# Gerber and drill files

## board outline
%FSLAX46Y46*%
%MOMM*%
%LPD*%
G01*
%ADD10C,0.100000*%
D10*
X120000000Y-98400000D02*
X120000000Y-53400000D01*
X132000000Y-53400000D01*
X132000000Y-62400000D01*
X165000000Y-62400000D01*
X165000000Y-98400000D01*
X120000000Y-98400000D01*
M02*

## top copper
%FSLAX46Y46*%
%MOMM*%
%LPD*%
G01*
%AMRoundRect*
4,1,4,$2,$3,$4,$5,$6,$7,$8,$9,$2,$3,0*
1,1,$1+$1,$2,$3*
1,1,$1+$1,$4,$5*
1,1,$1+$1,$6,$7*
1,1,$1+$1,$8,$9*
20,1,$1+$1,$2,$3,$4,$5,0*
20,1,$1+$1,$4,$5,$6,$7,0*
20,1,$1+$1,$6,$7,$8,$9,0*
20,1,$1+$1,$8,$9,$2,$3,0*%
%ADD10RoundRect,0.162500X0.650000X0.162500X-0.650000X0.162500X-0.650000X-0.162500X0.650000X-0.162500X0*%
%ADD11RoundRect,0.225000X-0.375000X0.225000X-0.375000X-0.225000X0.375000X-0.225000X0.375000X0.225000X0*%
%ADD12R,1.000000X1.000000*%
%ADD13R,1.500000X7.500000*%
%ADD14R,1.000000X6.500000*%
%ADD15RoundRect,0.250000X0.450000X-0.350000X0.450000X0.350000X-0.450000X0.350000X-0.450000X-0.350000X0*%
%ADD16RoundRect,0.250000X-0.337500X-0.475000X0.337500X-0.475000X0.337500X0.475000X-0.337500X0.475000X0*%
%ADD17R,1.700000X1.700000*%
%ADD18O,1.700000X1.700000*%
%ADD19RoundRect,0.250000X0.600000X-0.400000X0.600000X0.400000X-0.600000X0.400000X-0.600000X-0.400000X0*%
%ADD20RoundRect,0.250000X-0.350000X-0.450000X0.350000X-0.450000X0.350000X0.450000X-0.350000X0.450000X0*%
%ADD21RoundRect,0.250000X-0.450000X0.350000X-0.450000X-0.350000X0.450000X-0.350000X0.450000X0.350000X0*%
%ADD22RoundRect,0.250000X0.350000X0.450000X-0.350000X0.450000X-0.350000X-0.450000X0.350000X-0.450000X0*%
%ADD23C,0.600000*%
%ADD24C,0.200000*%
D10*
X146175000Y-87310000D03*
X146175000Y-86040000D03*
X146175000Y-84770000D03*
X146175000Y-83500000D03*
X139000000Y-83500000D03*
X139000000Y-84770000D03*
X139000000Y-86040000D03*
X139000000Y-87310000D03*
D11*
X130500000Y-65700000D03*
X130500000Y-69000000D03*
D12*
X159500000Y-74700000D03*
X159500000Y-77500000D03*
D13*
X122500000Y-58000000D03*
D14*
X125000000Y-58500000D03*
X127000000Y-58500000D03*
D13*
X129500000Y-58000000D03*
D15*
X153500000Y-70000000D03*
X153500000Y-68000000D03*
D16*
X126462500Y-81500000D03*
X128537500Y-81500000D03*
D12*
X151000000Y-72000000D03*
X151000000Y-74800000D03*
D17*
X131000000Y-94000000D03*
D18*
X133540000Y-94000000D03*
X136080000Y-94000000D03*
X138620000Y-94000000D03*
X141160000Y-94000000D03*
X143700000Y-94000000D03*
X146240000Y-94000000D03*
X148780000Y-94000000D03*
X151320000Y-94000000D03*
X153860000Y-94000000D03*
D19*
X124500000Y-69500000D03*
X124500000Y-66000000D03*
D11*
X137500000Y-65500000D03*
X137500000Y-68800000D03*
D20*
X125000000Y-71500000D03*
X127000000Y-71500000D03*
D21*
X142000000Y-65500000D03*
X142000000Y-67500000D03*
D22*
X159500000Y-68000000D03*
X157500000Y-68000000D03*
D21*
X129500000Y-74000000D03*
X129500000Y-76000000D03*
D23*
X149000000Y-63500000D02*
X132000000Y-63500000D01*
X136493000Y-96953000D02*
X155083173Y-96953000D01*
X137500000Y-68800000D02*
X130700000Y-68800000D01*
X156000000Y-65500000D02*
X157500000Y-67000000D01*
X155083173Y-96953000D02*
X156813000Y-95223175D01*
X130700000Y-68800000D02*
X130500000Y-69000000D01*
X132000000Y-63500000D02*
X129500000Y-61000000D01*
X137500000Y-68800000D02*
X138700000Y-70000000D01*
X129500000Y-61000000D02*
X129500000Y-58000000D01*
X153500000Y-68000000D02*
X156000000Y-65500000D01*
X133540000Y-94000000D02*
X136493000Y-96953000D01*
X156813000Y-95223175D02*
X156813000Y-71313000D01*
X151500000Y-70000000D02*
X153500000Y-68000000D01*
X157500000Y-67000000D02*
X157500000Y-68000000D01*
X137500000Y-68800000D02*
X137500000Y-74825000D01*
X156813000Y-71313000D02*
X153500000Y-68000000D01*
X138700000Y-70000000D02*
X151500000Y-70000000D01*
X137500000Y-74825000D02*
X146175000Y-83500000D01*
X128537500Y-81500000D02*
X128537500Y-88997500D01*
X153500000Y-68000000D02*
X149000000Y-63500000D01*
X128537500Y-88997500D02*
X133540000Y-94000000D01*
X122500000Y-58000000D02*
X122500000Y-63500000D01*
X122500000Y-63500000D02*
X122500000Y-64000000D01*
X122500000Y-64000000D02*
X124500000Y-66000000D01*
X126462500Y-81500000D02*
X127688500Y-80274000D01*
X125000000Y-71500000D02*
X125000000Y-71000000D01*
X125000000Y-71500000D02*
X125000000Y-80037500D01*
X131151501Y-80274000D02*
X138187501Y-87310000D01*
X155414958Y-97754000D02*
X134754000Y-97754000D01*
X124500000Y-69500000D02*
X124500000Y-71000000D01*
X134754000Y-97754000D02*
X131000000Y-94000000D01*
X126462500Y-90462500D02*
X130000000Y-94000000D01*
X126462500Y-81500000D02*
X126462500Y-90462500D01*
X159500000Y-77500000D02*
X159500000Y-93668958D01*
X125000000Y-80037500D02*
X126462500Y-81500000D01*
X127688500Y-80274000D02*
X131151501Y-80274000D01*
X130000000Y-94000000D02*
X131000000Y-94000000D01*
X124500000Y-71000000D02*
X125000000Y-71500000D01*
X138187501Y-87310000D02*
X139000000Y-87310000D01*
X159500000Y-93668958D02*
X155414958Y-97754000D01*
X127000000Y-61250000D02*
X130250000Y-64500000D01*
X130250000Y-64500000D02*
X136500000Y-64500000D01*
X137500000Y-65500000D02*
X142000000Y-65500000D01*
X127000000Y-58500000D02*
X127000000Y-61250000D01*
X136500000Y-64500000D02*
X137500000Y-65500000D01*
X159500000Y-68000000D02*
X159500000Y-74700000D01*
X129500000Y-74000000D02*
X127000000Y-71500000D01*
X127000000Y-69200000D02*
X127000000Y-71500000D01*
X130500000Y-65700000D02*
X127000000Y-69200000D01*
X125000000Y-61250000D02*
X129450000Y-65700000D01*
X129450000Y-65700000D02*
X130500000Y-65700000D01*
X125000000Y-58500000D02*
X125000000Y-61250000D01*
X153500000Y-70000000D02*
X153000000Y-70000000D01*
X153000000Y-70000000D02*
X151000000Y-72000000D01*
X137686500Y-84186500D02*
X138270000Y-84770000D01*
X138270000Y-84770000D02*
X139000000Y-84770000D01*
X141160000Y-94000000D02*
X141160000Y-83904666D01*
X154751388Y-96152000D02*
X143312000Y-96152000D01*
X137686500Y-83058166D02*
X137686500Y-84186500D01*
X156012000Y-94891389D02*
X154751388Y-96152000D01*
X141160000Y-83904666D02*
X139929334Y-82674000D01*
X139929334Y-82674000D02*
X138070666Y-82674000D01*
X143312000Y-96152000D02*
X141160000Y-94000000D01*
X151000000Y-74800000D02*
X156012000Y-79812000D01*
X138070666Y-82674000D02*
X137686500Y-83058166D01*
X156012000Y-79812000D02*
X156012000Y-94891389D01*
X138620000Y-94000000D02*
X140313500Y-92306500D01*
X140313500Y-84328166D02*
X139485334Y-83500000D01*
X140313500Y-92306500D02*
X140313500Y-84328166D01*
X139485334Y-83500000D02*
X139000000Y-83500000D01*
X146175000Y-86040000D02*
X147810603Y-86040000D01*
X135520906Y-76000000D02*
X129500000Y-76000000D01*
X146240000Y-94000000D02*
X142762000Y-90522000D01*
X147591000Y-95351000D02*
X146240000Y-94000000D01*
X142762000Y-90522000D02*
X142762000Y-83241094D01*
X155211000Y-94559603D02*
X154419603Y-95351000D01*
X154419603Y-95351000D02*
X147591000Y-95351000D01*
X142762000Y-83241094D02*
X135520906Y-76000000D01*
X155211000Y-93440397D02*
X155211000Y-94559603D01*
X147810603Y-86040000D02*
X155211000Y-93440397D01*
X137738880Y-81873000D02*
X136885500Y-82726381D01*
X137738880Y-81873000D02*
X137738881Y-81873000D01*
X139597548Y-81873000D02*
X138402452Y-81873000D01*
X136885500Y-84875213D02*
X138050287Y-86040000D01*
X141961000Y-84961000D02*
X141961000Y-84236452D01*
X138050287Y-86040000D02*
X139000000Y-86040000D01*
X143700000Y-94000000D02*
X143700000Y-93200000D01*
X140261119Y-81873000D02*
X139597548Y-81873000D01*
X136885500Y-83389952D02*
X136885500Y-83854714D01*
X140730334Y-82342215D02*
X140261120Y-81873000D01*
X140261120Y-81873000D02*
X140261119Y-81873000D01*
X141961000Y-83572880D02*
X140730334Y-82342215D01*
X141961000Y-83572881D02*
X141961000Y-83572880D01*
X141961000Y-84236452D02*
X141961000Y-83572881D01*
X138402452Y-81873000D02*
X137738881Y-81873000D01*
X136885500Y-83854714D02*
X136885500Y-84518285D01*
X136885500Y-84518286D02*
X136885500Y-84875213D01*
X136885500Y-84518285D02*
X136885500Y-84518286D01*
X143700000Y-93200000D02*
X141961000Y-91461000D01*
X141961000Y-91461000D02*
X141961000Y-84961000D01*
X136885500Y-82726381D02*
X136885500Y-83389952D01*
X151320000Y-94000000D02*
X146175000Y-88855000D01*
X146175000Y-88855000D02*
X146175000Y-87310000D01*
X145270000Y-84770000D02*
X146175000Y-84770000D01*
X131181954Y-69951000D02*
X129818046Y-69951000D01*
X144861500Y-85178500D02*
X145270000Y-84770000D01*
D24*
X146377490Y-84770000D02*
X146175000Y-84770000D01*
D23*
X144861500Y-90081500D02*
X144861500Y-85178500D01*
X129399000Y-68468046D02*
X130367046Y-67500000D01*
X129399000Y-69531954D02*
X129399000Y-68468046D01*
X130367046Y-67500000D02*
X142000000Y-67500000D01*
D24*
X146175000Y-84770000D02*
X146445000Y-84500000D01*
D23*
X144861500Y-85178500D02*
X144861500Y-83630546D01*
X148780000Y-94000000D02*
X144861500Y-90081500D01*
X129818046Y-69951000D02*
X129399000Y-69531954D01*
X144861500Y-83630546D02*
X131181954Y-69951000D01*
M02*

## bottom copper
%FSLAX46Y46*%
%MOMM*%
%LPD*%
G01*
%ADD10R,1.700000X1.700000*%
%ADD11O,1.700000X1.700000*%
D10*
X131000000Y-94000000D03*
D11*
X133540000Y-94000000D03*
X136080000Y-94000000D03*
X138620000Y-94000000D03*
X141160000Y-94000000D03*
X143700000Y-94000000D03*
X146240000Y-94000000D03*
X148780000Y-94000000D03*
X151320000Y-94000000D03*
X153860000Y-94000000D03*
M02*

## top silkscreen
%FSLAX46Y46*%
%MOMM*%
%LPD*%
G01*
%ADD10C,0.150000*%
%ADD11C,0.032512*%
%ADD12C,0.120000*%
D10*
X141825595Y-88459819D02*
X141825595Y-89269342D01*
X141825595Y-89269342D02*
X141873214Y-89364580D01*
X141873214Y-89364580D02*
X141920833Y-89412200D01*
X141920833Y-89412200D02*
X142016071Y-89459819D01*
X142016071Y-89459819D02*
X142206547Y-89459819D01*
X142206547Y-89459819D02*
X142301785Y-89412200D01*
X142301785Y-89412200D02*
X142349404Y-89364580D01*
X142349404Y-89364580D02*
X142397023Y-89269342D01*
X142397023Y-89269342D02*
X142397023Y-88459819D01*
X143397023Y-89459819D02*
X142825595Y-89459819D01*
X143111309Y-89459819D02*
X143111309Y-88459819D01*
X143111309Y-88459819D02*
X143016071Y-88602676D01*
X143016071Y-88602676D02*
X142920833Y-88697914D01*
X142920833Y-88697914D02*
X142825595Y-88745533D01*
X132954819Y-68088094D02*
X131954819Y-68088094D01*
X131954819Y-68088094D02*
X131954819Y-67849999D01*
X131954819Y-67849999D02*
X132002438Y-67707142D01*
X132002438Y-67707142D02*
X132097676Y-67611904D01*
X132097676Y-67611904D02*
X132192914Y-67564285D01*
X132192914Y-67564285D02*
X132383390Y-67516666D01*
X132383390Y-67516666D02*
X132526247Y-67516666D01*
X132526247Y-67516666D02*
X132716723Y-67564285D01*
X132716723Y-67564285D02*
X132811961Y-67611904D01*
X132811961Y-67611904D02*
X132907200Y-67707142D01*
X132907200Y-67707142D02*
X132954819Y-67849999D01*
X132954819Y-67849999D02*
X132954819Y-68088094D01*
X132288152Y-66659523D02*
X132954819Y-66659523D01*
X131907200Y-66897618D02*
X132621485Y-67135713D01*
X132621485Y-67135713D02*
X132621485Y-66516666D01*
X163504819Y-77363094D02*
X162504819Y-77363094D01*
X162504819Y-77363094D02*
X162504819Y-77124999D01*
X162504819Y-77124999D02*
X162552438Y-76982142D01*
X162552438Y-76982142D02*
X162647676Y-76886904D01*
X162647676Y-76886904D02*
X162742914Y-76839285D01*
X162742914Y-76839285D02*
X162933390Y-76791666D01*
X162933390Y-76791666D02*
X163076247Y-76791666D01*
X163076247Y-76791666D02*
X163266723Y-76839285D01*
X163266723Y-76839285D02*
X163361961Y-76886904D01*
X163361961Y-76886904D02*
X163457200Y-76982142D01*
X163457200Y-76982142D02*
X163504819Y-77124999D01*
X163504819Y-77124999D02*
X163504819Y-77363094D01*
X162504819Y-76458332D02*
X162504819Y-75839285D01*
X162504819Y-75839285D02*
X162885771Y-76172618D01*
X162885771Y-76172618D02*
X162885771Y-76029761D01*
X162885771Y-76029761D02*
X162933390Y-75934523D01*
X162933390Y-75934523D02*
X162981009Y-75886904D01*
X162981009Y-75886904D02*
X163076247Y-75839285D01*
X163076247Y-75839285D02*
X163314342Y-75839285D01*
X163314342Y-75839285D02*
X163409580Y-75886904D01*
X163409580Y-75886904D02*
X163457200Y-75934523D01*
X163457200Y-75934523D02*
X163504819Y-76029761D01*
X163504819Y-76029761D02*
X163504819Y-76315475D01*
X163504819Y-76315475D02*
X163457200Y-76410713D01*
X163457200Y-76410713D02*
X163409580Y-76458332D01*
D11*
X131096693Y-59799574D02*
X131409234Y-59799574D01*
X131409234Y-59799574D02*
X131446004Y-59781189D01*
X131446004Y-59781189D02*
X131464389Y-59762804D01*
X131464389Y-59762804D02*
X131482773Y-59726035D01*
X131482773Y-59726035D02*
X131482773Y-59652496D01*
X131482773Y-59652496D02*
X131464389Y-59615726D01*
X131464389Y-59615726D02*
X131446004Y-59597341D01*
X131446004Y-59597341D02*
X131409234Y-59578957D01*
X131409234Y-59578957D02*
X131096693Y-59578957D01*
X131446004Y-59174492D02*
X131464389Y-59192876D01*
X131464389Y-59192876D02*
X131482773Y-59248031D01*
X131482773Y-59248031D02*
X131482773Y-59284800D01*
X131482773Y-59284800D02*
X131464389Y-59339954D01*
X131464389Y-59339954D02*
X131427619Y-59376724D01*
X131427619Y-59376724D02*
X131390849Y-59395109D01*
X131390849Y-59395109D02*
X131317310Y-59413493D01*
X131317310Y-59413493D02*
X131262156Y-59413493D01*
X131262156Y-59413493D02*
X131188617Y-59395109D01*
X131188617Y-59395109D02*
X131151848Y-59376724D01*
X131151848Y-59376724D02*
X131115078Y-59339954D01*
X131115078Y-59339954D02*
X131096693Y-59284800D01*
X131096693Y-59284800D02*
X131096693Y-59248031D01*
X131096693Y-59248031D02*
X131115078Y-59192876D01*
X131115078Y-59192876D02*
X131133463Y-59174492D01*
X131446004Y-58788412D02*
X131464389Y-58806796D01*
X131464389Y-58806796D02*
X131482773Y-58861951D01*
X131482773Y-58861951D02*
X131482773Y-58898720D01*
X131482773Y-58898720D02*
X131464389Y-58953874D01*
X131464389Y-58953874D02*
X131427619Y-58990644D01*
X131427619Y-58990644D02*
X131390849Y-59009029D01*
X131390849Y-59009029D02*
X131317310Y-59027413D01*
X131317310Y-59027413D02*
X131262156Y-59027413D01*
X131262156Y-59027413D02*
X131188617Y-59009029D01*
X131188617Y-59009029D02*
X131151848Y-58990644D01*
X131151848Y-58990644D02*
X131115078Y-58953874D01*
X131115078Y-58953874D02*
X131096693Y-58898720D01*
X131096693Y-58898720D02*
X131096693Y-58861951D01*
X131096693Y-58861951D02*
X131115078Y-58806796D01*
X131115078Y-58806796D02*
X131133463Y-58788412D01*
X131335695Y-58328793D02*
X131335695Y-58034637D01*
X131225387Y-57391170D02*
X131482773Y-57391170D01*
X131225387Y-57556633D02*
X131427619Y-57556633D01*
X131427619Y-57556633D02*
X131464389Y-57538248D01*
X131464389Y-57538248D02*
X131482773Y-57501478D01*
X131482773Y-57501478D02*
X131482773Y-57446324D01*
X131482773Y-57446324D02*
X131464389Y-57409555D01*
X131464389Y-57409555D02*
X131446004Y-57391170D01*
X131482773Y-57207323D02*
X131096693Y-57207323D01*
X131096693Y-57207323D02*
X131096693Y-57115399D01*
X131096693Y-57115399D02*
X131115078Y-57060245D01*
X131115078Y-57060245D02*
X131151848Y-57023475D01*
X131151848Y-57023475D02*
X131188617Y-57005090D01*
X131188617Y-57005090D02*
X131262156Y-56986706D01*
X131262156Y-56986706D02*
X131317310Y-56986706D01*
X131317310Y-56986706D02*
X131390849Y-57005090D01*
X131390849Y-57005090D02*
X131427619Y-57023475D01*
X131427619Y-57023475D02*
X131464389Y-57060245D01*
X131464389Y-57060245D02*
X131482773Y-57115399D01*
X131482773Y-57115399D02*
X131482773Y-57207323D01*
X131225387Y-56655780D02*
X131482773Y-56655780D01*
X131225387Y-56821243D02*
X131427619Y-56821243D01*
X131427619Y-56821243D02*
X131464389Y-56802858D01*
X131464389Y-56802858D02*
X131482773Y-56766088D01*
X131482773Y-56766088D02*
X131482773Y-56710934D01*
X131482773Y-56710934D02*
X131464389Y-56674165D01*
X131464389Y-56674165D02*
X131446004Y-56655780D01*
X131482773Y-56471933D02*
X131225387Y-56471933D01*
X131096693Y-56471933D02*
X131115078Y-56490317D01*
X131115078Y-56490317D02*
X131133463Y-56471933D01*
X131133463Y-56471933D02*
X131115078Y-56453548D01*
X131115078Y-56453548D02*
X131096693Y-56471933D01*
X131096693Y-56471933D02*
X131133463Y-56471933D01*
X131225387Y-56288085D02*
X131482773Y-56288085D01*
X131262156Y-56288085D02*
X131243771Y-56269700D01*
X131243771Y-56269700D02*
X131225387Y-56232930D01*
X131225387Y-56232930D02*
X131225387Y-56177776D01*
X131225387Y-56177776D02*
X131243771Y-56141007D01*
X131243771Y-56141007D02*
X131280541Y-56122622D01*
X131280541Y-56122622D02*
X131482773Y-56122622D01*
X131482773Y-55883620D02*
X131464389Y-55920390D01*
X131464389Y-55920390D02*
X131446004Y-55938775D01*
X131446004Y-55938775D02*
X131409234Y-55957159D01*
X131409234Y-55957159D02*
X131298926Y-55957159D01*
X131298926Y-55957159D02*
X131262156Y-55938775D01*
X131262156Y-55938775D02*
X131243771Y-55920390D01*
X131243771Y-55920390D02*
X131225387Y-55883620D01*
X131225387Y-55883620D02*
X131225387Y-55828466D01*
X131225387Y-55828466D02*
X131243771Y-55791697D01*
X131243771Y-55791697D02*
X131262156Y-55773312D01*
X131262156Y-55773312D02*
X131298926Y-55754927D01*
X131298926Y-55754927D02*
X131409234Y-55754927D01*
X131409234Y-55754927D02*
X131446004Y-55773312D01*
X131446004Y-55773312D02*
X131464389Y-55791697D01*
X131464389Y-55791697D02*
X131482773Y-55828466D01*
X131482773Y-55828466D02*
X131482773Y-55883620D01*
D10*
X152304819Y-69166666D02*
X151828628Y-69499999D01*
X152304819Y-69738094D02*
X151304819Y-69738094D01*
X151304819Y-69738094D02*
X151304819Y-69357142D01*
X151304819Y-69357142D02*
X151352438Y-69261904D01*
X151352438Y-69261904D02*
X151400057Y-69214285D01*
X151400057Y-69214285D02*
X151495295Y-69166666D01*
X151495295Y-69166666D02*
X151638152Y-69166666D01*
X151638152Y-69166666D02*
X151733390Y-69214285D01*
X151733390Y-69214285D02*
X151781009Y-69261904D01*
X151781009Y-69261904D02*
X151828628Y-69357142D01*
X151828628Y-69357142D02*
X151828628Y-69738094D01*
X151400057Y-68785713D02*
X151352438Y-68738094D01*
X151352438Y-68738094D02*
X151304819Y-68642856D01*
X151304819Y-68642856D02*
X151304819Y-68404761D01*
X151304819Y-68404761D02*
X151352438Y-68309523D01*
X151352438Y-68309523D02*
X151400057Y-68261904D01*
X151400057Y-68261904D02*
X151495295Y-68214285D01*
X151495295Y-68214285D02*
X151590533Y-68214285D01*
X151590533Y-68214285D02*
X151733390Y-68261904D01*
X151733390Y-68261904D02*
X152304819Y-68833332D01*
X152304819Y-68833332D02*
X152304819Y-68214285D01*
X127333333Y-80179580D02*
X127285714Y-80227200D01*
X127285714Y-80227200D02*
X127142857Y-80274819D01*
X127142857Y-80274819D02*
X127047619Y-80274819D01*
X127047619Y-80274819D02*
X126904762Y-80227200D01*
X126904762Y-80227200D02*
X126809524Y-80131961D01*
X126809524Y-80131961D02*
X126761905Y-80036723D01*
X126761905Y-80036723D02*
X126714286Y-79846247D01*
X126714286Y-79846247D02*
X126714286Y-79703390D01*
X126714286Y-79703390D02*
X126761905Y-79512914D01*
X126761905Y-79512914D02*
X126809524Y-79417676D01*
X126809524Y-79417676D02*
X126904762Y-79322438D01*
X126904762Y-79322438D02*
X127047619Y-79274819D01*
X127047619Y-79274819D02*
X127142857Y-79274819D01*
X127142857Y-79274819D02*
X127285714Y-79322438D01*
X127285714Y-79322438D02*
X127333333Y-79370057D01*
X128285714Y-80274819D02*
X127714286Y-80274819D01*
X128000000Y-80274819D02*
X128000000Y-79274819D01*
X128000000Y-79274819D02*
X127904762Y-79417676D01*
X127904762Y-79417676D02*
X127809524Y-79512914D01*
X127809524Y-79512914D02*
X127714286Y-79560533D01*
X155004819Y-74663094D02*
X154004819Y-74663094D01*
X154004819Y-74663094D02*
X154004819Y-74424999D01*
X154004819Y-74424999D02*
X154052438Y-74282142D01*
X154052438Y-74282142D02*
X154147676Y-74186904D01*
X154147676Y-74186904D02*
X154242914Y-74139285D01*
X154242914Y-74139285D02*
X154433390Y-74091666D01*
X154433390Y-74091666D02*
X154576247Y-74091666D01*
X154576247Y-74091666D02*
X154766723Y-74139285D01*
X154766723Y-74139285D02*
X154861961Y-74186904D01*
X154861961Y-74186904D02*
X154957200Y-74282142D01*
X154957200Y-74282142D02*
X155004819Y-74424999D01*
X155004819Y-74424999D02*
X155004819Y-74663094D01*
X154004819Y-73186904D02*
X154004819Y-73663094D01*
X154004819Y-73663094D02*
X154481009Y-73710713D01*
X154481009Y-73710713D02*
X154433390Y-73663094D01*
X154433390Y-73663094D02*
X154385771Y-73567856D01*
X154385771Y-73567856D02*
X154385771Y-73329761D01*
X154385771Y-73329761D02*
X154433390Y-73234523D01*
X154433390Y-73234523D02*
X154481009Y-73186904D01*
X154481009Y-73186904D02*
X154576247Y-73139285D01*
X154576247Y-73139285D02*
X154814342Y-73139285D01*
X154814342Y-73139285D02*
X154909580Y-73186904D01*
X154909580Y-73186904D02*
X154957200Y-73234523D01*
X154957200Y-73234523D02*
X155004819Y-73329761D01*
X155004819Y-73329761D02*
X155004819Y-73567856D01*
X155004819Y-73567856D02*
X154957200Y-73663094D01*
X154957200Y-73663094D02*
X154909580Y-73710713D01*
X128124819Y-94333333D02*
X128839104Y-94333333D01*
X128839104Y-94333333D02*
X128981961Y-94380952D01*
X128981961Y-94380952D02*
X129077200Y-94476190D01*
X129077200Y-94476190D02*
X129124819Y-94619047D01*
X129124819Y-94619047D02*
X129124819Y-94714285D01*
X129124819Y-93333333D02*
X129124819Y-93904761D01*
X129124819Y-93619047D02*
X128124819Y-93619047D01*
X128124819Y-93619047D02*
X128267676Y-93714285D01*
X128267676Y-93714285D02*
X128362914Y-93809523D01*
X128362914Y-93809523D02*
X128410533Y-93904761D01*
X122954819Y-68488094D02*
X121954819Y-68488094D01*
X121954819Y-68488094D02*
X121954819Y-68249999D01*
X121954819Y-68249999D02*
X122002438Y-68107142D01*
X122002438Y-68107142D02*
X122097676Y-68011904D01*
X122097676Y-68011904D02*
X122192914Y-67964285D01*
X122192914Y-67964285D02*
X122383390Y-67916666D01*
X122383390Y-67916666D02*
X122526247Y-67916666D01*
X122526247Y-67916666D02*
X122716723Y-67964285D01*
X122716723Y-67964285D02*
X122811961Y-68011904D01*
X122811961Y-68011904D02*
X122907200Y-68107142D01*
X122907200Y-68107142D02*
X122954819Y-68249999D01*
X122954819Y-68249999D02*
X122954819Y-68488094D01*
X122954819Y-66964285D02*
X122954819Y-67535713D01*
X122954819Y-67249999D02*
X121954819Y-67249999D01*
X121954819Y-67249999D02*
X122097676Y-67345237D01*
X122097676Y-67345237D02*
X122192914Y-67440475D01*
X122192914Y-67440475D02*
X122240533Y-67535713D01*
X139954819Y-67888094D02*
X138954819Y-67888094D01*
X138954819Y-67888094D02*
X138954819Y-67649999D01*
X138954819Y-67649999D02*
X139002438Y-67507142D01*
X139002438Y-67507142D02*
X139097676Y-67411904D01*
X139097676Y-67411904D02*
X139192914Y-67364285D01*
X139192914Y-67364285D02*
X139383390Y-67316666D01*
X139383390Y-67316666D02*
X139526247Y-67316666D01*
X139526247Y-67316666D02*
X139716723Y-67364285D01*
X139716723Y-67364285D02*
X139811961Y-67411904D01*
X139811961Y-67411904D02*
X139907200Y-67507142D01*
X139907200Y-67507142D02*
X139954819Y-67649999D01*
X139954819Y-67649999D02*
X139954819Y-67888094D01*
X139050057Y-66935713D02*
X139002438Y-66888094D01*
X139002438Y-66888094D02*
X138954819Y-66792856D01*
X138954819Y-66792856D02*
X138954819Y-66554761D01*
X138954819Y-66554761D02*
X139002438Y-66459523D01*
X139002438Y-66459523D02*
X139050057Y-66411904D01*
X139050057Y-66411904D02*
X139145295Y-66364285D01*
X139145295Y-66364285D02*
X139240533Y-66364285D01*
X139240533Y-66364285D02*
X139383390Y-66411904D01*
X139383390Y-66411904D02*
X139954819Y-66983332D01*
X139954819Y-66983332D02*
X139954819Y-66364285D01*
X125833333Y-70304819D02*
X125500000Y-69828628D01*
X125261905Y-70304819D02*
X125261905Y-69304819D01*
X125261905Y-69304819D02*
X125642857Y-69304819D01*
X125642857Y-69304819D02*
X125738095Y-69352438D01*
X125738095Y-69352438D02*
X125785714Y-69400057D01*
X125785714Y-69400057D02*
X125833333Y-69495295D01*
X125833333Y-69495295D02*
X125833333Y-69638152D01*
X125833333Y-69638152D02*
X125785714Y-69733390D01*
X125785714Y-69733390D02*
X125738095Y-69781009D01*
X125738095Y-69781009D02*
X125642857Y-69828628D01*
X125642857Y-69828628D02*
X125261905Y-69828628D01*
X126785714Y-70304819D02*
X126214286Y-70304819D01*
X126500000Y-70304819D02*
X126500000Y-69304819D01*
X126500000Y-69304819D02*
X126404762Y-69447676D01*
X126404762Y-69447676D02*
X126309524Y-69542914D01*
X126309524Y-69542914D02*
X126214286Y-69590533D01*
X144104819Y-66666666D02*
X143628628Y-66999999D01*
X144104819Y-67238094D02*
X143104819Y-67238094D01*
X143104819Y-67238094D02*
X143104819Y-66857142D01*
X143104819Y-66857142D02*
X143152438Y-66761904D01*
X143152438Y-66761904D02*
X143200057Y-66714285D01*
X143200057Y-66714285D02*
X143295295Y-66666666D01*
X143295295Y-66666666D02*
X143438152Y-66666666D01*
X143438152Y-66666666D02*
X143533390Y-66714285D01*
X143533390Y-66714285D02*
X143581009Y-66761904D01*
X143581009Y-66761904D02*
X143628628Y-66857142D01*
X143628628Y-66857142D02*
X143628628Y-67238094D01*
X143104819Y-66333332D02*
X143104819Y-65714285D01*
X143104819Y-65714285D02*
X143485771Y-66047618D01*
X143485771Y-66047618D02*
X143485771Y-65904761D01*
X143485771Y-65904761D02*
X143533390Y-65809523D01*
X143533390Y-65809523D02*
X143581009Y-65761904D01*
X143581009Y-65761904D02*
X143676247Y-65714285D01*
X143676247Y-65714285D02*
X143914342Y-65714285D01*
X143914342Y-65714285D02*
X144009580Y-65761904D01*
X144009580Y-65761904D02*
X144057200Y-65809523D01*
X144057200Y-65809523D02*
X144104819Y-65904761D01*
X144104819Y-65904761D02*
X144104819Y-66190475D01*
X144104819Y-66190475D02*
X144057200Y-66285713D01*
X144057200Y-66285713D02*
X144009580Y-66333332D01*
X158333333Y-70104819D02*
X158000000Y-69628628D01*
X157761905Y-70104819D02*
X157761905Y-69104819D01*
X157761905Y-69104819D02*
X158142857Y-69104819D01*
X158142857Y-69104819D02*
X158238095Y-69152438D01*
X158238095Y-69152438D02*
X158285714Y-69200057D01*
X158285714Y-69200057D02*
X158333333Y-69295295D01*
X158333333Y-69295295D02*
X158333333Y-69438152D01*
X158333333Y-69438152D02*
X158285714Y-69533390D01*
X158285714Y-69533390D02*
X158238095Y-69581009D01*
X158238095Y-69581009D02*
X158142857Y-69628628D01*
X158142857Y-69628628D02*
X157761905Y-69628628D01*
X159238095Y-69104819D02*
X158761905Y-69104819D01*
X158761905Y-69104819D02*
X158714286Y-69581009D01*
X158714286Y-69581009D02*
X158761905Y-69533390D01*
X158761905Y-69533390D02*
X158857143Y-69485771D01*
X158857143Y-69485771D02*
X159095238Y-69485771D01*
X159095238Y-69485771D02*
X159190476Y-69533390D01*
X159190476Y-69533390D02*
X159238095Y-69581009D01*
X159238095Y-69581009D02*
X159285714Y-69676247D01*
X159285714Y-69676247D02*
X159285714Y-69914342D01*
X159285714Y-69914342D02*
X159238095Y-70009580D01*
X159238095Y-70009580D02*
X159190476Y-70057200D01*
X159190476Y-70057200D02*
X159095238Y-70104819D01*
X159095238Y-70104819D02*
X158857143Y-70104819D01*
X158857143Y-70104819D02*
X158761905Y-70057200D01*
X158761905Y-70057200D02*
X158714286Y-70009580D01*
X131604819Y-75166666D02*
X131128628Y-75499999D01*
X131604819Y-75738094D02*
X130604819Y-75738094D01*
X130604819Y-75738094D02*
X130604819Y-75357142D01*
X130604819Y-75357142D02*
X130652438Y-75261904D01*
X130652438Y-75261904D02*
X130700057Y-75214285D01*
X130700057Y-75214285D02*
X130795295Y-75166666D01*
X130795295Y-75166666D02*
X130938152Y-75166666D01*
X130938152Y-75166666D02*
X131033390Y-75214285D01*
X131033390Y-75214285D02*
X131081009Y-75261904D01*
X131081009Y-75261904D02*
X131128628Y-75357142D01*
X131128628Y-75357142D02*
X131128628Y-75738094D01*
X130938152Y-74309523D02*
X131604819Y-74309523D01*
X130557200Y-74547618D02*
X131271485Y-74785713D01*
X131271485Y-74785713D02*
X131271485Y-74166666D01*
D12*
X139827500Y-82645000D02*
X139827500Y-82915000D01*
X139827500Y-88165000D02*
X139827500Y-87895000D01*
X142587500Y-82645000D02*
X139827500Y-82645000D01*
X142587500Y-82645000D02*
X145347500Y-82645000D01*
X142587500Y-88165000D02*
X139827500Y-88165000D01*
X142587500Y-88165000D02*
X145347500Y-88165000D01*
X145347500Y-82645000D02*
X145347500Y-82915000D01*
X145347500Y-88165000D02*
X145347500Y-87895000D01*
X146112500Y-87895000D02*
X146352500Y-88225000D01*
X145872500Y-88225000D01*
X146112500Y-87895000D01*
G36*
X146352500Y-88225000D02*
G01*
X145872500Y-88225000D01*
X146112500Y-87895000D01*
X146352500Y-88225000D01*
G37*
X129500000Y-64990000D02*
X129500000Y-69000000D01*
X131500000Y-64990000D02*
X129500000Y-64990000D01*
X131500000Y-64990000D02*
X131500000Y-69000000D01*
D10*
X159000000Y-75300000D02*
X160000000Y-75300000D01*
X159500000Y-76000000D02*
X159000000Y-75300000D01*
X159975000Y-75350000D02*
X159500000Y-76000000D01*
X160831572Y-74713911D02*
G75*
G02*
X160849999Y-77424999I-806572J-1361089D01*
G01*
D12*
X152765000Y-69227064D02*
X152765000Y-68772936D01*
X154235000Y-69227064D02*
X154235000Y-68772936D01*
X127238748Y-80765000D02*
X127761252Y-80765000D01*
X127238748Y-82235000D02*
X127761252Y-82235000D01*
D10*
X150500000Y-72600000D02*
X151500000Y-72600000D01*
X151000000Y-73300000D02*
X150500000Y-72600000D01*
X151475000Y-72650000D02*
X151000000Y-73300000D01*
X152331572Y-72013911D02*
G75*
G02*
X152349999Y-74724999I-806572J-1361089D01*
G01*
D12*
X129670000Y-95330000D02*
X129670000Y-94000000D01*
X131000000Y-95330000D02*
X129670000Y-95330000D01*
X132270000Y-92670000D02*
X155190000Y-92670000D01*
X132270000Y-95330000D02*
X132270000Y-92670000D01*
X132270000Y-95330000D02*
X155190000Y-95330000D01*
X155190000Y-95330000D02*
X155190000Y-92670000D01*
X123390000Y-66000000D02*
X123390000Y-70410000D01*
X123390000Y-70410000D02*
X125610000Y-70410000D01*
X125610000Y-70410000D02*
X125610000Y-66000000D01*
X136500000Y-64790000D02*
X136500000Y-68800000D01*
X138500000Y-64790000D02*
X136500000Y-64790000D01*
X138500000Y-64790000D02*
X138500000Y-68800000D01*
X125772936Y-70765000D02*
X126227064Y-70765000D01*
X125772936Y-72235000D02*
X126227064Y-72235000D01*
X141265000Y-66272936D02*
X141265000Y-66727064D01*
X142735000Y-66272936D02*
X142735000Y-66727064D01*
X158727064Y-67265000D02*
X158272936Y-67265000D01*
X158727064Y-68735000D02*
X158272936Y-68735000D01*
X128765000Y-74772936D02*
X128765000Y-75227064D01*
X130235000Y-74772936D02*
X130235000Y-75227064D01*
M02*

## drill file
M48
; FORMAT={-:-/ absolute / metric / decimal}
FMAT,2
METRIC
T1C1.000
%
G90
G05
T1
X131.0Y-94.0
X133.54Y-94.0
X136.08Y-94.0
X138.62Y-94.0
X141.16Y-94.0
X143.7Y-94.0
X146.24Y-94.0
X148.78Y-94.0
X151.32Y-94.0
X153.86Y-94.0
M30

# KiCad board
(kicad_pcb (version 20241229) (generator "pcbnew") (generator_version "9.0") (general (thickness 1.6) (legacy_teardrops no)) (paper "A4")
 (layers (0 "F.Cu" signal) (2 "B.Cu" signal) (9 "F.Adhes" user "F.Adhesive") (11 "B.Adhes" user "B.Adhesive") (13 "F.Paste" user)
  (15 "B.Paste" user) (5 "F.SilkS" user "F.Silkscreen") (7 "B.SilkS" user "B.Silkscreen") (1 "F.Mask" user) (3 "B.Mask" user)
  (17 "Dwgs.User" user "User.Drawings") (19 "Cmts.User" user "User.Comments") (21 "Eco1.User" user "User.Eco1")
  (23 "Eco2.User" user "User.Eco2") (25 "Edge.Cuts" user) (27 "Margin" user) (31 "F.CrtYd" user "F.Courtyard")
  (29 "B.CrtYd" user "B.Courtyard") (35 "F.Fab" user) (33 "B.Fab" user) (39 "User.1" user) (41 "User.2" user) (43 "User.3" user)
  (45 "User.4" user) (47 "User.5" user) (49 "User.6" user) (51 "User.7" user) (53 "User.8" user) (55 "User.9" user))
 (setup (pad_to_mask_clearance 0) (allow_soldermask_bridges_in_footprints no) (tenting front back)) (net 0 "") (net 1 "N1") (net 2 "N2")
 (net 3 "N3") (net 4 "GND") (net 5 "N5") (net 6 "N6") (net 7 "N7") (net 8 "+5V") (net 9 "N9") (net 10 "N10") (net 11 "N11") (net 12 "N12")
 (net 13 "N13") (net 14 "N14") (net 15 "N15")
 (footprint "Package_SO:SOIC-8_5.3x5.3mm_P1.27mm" (layer "F.Cu") (at 142.5875 85.405 180)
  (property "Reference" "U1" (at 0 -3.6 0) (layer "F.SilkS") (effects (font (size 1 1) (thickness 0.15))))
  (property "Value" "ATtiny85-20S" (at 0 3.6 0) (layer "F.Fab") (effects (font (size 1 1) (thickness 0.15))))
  (fp_line (start 2.76 2.76) (end 2.76 2.49) (stroke (width 0.12) (type solid)) (layer "F.SilkS"))
  (fp_line (start 2.76 -2.76) (end 2.76 -2.49) (stroke (width 0.12) (type solid)) (layer "F.SilkS"))
  (fp_line (start 0 2.76) (end 2.76 2.76) (stroke (width 0.12) (type solid)) (layer "F.SilkS"))
  (fp_line (start 0 2.76) (end -2.76 2.76) (stroke (width 0.12) (type solid)) (layer "F.SilkS"))
  (fp_line (start 0 -2.76) (end 2.76 -2.76) (stroke (width 0.12) (type solid)) (layer "F.SilkS"))
  (fp_line (start 0 -2.76) (end -2.76 -2.76) (stroke (width 0.12) (type solid)) (layer "F.SilkS"))
  (fp_line (start -2.76 2.76) (end -2.76 2.49) (stroke (width 0.12) (type solid)) (layer "F.SilkS"))
  (fp_line (start -2.76 -2.76) (end -2.76 -2.49) (stroke (width 0.12) (type solid)) (layer "F.SilkS"))
  (fp_poly (pts (xy -3.525 -2.49) (xy -3.765 -2.82) (xy -3.285 -2.82)) (stroke (width 0.12) (type solid)) (fill yes) (layer "F.SilkS"))
  (pad "1" smd roundrect (at -3.5875 -1.905 180) (size 1.625 0.65) (layers "F.Cu" "F.Mask" "F.Paste") (roundrect_rratio 0.25) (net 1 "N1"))
  (pad "2" smd roundrect (at -3.5875 -0.635 180) (size 1.625 0.65) (layers "F.Cu" "F.Mask" "F.Paste") (roundrect_rratio 0.25) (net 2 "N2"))
  (pad "3" smd roundrect (at -3.5875 0.635 180) (size 1.625 0.65) (layers "F.Cu" "F.Mask" "F.Paste") (roundrect_rratio 0.25) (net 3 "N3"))
  (pad "4" smd roundrect (at -3.5875 1.905 180) (size 1.625 0.65) (layers "F.Cu" "F.Mask" "F.Paste") (roundrect_rratio 0.25) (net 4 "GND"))
  (pad "5" smd roundrect (at 3.5875 1.905 180) (size 1.625 0.65) (layers "F.Cu" "F.Mask" "F.Paste") (roundrect_rratio 0.25) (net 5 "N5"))
  (pad "6" smd roundrect (at 3.5875 0.635 180) (size 1.625 0.65) (layers "F.Cu" "F.Mask" "F.Paste") (roundrect_rratio 0.25) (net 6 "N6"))
  (pad "7" smd roundrect (at 3.5875 -0.635 180) (size 1.625 0.65) (layers "F.Cu" "F.Mask" "F.Paste") (roundrect_rratio 0.25) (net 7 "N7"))
  (pad "8" smd roundrect (at 3.5875 -1.905 180) (size 1.625 0.65) (layers "F.Cu" "F.Mask" "F.Paste") (roundrect_rratio 0.25) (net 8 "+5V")))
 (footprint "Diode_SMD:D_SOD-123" (layer "F.Cu") (at 130.5 67.35 -90)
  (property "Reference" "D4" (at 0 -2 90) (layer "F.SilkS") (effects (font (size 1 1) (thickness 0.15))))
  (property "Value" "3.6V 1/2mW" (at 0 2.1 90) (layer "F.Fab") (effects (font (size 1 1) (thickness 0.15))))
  (fp_line (start -2.36 1) (end 1.65 1) (stroke (width 0.12) (type solid)) (layer "F.SilkS"))
  (fp_line (start -2.36 -1) (end -2.36 1) (stroke (width 0.12) (type solid)) (layer "F.SilkS"))
  (fp_line (start -2.36 -1) (end 1.65 -1) (stroke (width 0.12) (type solid)) (layer "F.SilkS"))
  (pad "1" smd roundrect (at -1.65 0 270) (size 0.9 1.2) (layers "F.Cu" "F.Mask" "F.Paste") (roundrect_rratio 0.25) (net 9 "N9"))
  (pad "2" smd roundrect (at 1.65 0 270) (size 0.9 1.2) (layers "F.Cu" "F.Mask" "F.Paste") (roundrect_rratio 0.25) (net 4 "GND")))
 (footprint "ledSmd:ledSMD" (layer "F.Cu") (at 159.5 76.5 -90)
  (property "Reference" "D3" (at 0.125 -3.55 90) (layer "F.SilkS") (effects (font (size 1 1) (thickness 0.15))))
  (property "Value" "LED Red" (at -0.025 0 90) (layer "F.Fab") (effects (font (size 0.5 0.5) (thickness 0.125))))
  (fp_line (start -1.2 0.5) (end -1.2 -0.5) (stroke (width 0.15) (type solid)) (layer "F.SilkS"))
  (fp_line (start -0.5 0) (end -1.2 0.5) (stroke (width 0.15) (type solid)) (layer "F.SilkS"))
  (fp_line (start -1.15 -0.475) (end -0.5 0) (stroke (width 0.15) (type solid)) (layer "F.SilkS"))
  (fp_arc (start -1.786089 -1.331572) (mid -0.435753 -2.107089) (end 0.924999 -1.349999) (stroke (width 0.15) (type solid))
   (layer "F.SilkS"))
  (pad "1" smd rect (at -1.8 0 270) (size 1 1) (layers "F.Cu" "F.Mask" "F.Paste") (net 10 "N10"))
  (pad "2" smd rect (at 1 0 270) (size 1 1) (layers "F.Cu" "F.Mask" "F.Paste") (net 8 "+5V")))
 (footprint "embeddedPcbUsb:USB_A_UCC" (layer "F.Cu") (at 126 58.2 -90)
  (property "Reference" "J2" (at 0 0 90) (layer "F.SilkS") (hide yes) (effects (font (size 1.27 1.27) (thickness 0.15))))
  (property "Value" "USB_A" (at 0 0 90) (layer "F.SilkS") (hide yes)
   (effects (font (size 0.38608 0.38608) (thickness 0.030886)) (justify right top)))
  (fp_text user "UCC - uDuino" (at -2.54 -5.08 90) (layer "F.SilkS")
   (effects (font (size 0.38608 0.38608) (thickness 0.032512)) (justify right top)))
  (pad "1" smd rect (at -0.2 3.5 270) (size 7.5 1.5) (layers "F.Cu" "F.Mask" "F.Paste") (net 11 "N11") (solder_mask_margin 0.1016))
  (pad "2" smd rect (at 0.3 1 270) (size 6.5 1) (layers "F.Cu" "F.Mask" "F.Paste") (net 9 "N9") (solder_mask_margin 0.1016))
  (pad "3" smd rect (at 0.3 -1 270) (size 6.5 1) (layers "F.Cu" "F.Mask" "F.Paste") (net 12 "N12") (solder_mask_margin 0.1016))
  (pad "4" smd rect (at -0.2 -3.5 270) (size 7.5 1.5) (layers "F.Cu" "F.Mask" "F.Paste") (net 4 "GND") (solder_mask_margin 0.1016)))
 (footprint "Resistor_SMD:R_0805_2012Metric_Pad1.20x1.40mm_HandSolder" (layer "F.Cu") (at 153.5 69 90)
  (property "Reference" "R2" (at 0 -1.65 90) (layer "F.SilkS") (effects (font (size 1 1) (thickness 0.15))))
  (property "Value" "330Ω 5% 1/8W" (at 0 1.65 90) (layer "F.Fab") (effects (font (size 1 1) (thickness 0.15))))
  (fp_line (start -0.227064 -0.735) (end 0.227064 -0.735) (stroke (width 0.12) (type solid)) (layer "F.SilkS"))
  (fp_line (start -0.227064 0.735) (end 0.227064 0.735) (stroke (width 0.12) (type solid)) (layer "F.SilkS"))
  (pad "1" smd roundrect (at -1 0 90) (size 1.2 1.4) (layers "F.Cu" "F.Mask" "F.Paste") (roundrect_rratio 0.208333) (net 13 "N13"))
  (pad "2" smd roundrect (at 1 0 90) (size 1.2 1.4) (layers "F.Cu" "F.Mask" "F.Paste") (roundrect_rratio 0.208333) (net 4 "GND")))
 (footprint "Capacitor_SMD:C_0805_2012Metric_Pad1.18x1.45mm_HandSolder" (layer "F.Cu") (at 127.5 81.5)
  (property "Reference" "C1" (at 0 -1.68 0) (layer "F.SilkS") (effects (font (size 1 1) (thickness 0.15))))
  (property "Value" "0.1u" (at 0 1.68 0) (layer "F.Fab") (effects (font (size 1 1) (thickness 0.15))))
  (fp_line (start -0.261252 -0.735) (end 0.261252 -0.735) (stroke (width 0.12) (type solid)) (layer "F.SilkS"))
  (fp_line (start -0.261252 0.735) (end 0.261252 0.735) (stroke (width 0.12) (type solid)) (layer "F.SilkS"))
  (pad "1" smd roundrect (at -1.0375 0) (size 1.175 1.45) (layers "F.Cu" "F.Mask" "F.Paste") (roundrect_rratio 0.212766) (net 8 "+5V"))
  (pad "2" smd roundrect (at 1.0375 0) (size 1.175 1.45) (layers "F.Cu" "F.Mask" "F.Paste") (roundrect_rratio 0.212766) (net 4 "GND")))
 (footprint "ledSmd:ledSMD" (layer "F.Cu") (at 151 73.8 -90)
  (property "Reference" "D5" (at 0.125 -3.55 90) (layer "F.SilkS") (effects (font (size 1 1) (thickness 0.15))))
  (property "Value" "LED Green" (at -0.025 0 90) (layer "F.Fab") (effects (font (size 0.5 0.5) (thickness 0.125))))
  (fp_line (start -1.2 0.5) (end -1.2 -0.5) (stroke (width 0.15) (type solid)) (layer "F.SilkS"))
  (fp_line (start -0.5 0) (end -1.2 0.5) (stroke (width 0.15) (type solid)) (layer "F.SilkS"))
  (fp_line (start -1.15 -0.475) (end -0.5 0) (stroke (width 0.15) (type solid)) (layer "F.SilkS"))
  (fp_arc (start -1.786089 -1.331572) (mid -0.435753 -2.107089) (end 0.924999 -1.349999) (stroke (width 0.15) (type solid))
   (layer "F.SilkS"))
  (pad "1" smd rect (at -1.8 0 270) (size 1 1) (layers "F.Cu" "F.Mask" "F.Paste") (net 13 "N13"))
  (pad "2" smd rect (at 1 0 270) (size 1 1) (layers "F.Cu" "F.Mask" "F.Paste") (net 6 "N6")))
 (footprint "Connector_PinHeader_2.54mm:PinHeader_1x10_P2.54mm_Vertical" (layer "F.Cu") (at 131 94 90)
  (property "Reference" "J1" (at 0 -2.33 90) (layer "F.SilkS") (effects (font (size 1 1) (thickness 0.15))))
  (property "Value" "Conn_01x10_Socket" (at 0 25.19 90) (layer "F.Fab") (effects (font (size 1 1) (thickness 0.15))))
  (fp_line (start -1.33 -1.33) (end 0 -1.33) (stroke (width 0.12) (type solid)) (layer "F.SilkS"))
  (fp_line (start -1.33 0) (end -1.33 -1.33) (stroke (width 0.12) (type solid)) (layer "F.SilkS"))
  (fp_line (start 1.33 1.27) (end 1.33 24.19) (stroke (width 0.12) (type solid)) (layer "F.SilkS"))
  (fp_line (start -1.33 1.27) (end 1.33 1.27) (stroke (width 0.12) (type solid)) (layer "F.SilkS"))
  (fp_line (start -1.33 1.27) (end -1.33 24.19) (stroke (width 0.12) (type solid)) (layer "F.SilkS"))
  (fp_line (start -1.33 24.19) (end 1.33 24.19) (stroke (width 0.12) (type solid)) (layer "F.SilkS"))
  (pad "1" thru_hole rect (at 0 0 90) (size 1.7 1.7) (drill 1) (layers "*.Cu" "*.Mask") (remove_unused_layers no) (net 8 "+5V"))
  (pad "2" thru_hole oval (at 0 2.54 90) (size 1.7 1.7) (drill 1) (layers "*.Cu" "*.Mask") (remove_unused_layers no) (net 4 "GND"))
  (pad "3" thru_hole oval (at 0 5.08 90) (size 1.7 1.7) (drill 1) (layers "*.Cu" "*.Mask") (remove_unused_layers no) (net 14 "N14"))
  (pad "4" thru_hole oval (at 0 7.62 90) (size 1.7 1.7) (drill 1) (layers "*.Cu" "*.Mask") (remove_unused_layers no) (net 5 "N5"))
  (pad "5" thru_hole oval (at 0 10.16 90) (size 1.7 1.7) (drill 1) (layers "*.Cu" "*.Mask") (remove_unused_layers no) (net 6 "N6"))
  (pad "6" thru_hole oval (at 0 12.7 90) (size 1.7 1.7) (drill 1) (layers "*.Cu" "*.Mask") (remove_unused_layers no) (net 7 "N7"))
  (pad "7" thru_hole oval (at 0 15.24 90) (size 1.7 1.7) (drill 1) (layers "*.Cu" "*.Mask") (remove_unused_layers no) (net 2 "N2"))
  (pad "8" thru_hole oval (at 0 17.78 90) (size 1.7 1.7) (drill 1) (layers "*.Cu" "*.Mask") (remove_unused_layers no) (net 3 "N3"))
  (pad "9" thru_hole oval (at 0 20.32 90) (size 1.7 1.7) (drill 1) (layers "*.Cu" "*.Mask") (remove_unused_layers no) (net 1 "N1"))
  (pad "10" thru_hole oval (at 0 22.86 90) (size 1.7 1.7) (drill 1) (layers "*.Cu" "*.Mask") (remove_unused_layers no) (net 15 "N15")))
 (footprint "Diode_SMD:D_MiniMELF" (layer "F.Cu") (at 124.5 67.75 90)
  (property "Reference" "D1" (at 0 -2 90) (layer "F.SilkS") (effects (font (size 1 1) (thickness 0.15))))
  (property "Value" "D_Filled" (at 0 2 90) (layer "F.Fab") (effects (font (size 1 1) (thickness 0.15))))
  (fp_line (start 1.75 -1.11) (end -2.66 -1.11) (stroke (width 0.12) (type solid)) (layer "F.SilkS"))
  (fp_line (start -2.66 -1.11) (end -2.66 1.11) (stroke (width 0.12) (type solid)) (layer "F.SilkS"))
  (fp_line (start -2.66 1.11) (end 1.75 1.11) (stroke (width 0.12) (type solid)) (layer "F.SilkS"))
  (pad "1" smd roundrect (at -1.75 0 90) (size 1.3 1.7) (layers "F.Cu" "F.Mask" "F.Paste") (roundrect_rratio 0.1923076923) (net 8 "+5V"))
  (pad "2" smd roundrect (at 1.75 0 90) (size 1.3 1.7) (layers "F.Cu" "F.Mask" "F.Paste") (roundrect_rratio 0.1923076923) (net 11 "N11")))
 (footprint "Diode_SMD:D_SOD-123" (layer "F.Cu") (at 137.5 67.15 -90)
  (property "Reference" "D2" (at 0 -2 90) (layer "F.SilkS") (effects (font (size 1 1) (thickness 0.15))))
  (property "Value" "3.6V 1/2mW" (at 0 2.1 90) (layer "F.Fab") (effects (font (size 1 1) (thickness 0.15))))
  (fp_line (start -2.36 1) (end 1.65 1) (stroke (width 0.12) (type solid)) (layer "F.SilkS"))
  (fp_line (start -2.36 -1) (end -2.36 1) (stroke (width 0.12) (type solid)) (layer "F.SilkS"))
  (fp_line (start -2.36 -1) (end 1.65 -1) (stroke (width 0.12) (type solid)) (layer "F.SilkS"))
  (pad "1" smd roundrect (at -1.65 0 270) (size 0.9 1.2) (layers "F.Cu" "F.Mask" "F.Paste") (roundrect_rratio 0.25) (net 12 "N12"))
  (pad "2" smd roundrect (at 1.65 0 270) (size 0.9 1.2) (layers "F.Cu" "F.Mask" "F.Paste") (roundrect_rratio 0.25) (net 4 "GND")))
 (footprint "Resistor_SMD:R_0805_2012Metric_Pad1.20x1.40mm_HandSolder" (layer "F.Cu") (at 126 71.5)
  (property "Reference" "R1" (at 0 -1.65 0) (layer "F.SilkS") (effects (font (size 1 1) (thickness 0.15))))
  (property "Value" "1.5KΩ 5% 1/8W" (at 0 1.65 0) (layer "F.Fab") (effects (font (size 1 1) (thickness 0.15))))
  (fp_line (start -0.227064 -0.735) (end 0.227064 -0.735) (stroke (width 0.12) (type solid)) (layer "F.SilkS"))
  (fp_line (start -0.227064 0.735) (end 0.227064 0.735) (stroke (width 0.12) (type solid)) (layer "F.SilkS"))
  (pad "1" smd roundrect (at -1 0) (size 1.2 1.4) (layers "F.Cu" "F.Mask" "F.Paste") (roundrect_rratio 0.208333) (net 8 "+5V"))
  (pad "2" smd roundrect (at 1 0) (size 1.2 1.4) (layers "F.Cu" "F.Mask" "F.Paste") (roundrect_rratio 0.208333) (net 9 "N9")))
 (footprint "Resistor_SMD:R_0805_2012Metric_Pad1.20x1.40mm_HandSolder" (layer "F.Cu") (at 142 66.5 -90)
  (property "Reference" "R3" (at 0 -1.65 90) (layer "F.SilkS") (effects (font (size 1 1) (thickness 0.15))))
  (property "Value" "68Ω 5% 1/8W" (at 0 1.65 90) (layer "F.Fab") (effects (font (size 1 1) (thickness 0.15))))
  (fp_line (start -0.227064 0.735) (end 0.227064 0.735) (stroke (width 0.12) (type solid)) (layer "F.SilkS"))
  (fp_line (start -0.227064 -0.735) (end 0.227064 -0.735) (stroke (width 0.12) (type solid)) (layer "F.SilkS"))
  (pad "1" smd roundrect (at -1 0 270) (size 1.2 1.4) (layers "F.Cu" "F.Mask" "F.Paste") (roundrect_rratio 0.208333) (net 12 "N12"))
  (pad "2" smd roundrect (at 1 0 270) (size 1.2 1.4) (layers "F.Cu" "F.Mask" "F.Paste") (roundrect_rratio 0.208333) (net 3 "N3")))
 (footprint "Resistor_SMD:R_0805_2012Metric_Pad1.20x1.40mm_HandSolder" (layer "F.Cu") (at 158.5 68 180)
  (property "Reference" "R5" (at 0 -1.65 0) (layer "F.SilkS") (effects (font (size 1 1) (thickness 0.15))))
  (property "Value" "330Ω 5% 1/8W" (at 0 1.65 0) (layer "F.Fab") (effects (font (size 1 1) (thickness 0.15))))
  (fp_line (start -0.227064 0.735) (end 0.227064 0.735) (stroke (width 0.12) (type solid)) (layer "F.SilkS"))
  (fp_line (start -0.227064 -0.735) (end 0.227064 -0.735) (stroke (width 0.12) (type solid)) (layer "F.SilkS"))
  (pad "1" smd roundrect (at -1 0 180) (size 1.2 1.4) (layers "F.Cu" "F.Mask" "F.Paste") (roundrect_rratio 0.208333) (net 10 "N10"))
  (pad "2" smd roundrect (at 1 0 180) (size 1.2 1.4) (layers "F.Cu" "F.Mask" "F.Paste") (roundrect_rratio 0.208333) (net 4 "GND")))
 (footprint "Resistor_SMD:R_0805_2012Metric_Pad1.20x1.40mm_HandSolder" (layer "F.Cu") (at 129.5 75 -90)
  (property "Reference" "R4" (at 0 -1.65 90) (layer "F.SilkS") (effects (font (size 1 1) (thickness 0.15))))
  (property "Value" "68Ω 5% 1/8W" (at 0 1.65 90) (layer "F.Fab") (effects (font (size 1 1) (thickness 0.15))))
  (fp_line (start -0.227064 0.735) (end 0.227064 0.735) (stroke (width 0.12) (type solid)) (layer "F.SilkS"))
  (fp_line (start -0.227064 -0.735) (end 0.227064 -0.735) (stroke (width 0.12) (type solid)) (layer "F.SilkS"))
  (pad "1" smd roundrect (at -1 0 270) (size 1.2 1.4) (layers "F.Cu" "F.Mask" "F.Paste") (roundrect_rratio 0.208333) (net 9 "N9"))
  (pad "2" smd roundrect (at 1 0 270) (size 1.2 1.4) (layers "F.Cu" "F.Mask" "F.Paste") (roundrect_rratio 0.208333) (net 2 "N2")))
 (gr_poly
  (pts (xy 120 98.4) (xy 120 53.4) (xy 132 53.4) (xy 132 62.4) (xy 165 62.4) (xy 165 98.4)) (stroke (width 0.1) (type solid)) (fill no)
  (layer "Edge.Cuts"))
 (segment (start 149 63.5) (end 132 63.5) (width 0.6) (layer "F.Cu") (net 4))
 (segment (start 136.493 96.953) (end 155.083173 96.953) (width 0.6) (layer "F.Cu") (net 4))
 (segment (start 137.5 68.8) (end 130.7 68.8) (width 0.6) (layer "F.Cu") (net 4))
 (segment (start 156 65.5) (end 157.5 67) (width 0.6) (layer "F.Cu") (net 4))
 (segment (start 155.083173 96.953) (end 156.813 95.223175) (width 0.6) (layer "F.Cu") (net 4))
 (segment (start 130.7 68.8) (end 130.5 69) (width 0.6) (layer "F.Cu") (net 4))
 (segment (start 132 63.5) (end 129.5 61) (width 0.6) (layer "F.Cu") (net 4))
 (segment (start 137.5 68.8) (end 138.7 70) (width 0.6) (layer "F.Cu") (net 4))
 (segment (start 129.5 61) (end 129.5 58) (width 0.6) (layer "F.Cu") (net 4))
 (segment (start 153.5 68) (end 156 65.5) (width 0.6) (layer "F.Cu") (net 4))
 (segment (start 133.54 94) (end 136.493 96.953) (width 0.6) (layer "F.Cu") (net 4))
 (segment (start 156.813 95.223175) (end 156.813 71.313) (width 0.6) (layer "F.Cu") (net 4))
 (segment (start 151.5 70) (end 153.5 68) (width 0.6) (layer "F.Cu") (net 4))
 (segment (start 157.5 67) (end 157.5 68) (width 0.6) (layer "F.Cu") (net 4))
 (segment (start 137.5 68.8) (end 137.5 74.825) (width 0.6) (layer "F.Cu") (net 4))
 (segment (start 156.813 71.313) (end 153.5 68) (width 0.6) (layer "F.Cu") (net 4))
 (segment (start 138.7 70) (end 151.5 70) (width 0.6) (layer "F.Cu") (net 4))
 (segment (start 137.5 74.825) (end 146.175 83.5) (width 0.6) (layer "F.Cu") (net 4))
 (segment (start 128.5375 81.5) (end 128.5375 88.9975) (width 0.6) (layer "F.Cu") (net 4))
 (segment (start 153.5 68) (end 149 63.5) (width 0.6) (layer "F.Cu") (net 4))
 (segment (start 128.5375 88.9975) (end 133.54 94) (width 0.6) (layer "F.Cu") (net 4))
 (segment (start 122.5 58) (end 122.5 63.5) (width 0.6) (layer "F.Cu") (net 11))
 (segment (start 122.5 63.5) (end 122.5 64) (width 0.6) (layer "F.Cu") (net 11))
 (segment (start 122.5 64) (end 124.5 66) (width 0.6) (layer "F.Cu") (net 11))
 (segment (start 126.4625 81.5) (end 127.6885 80.274) (width 0.6) (layer "F.Cu") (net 8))
 (segment (start 125 71.5) (end 125 71) (width 0.6) (layer "F.Cu") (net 8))
 (segment (start 125 71.5) (end 125 80.0375) (width 0.6) (layer "F.Cu") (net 8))
 (segment (start 131.151501 80.274) (end 138.187501 87.31) (width 0.6) (layer "F.Cu") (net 8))
 (segment (start 155.414958 97.754) (end 134.754 97.754) (width 0.6) (layer "F.Cu") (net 8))
 (segment (start 124.5 69.5) (end 124.5 71) (width 0.6) (layer "F.Cu") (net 8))
 (segment (start 134.754 97.754) (end 131 94) (width 0.6) (layer "F.Cu") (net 8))
 (segment (start 126.4625 90.4625) (end 130 94) (width 0.6) (layer "F.Cu") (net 8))
 (segment (start 126.4625 81.5) (end 126.4625 90.4625) (width 0.6) (layer "F.Cu") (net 8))
 (segment (start 159.5 77.5) (end 159.5 93.668958) (width 0.6) (layer "F.Cu") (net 8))
 (segment (start 125 80.0375) (end 126.4625 81.5) (width 0.6) (layer "F.Cu") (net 8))
 (segment (start 127.6885 80.274) (end 131.151501 80.274) (width 0.6) (layer "F.Cu") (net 8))
 (segment (start 130 94) (end 131 94) (width 0.6) (layer "F.Cu") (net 8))
 (segment (start 124.5 71) (end 125 71.5) (width 0.6) (layer "F.Cu") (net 8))
 (segment (start 138.187501 87.31) (end 139 87.31) (width 0.6) (layer "F.Cu") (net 8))
 (segment (start 159.5 93.668958) (end 155.414958 97.754) (width 0.6) (layer "F.Cu") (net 8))
 (segment (start 127 61.25) (end 130.25 64.5) (width 0.6) (layer "F.Cu") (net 12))
 (segment (start 130.25 64.5) (end 136.5 64.5) (width 0.6) (layer "F.Cu") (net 12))
 (segment (start 137.5 65.5) (end 142 65.5) (width 0.6) (layer "F.Cu") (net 12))
 (segment (start 127 58.5) (end 127 61.25) (width 0.6) (layer "F.Cu") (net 12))
 (segment (start 136.5 64.5) (end 137.5 65.5) (width 0.6) (layer "F.Cu") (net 12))
 (segment (start 159.5 68) (end 159.5 74.7) (width 0.6) (layer "F.Cu") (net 10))
 (segment (start 129.5 74) (end 127 71.5) (width 0.6) (layer "F.Cu") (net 9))
 (segment (start 127 69.2) (end 127 71.5) (width 0.6) (layer "F.Cu") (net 9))
 (segment (start 130.5 65.7) (end 127 69.2) (width 0.6) (layer "F.Cu") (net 9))
 (segment (start 125 61.25) (end 129.45 65.7) (width 0.6) (layer "F.Cu") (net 9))
 (segment (start 129.45 65.7) (end 130.5 65.7) (width 0.6) (layer "F.Cu") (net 9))
 (segment (start 125 58.5) (end 125 61.25) (width 0.6) (layer "F.Cu") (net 9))
 (segment (start 153.5 70) (end 153 70) (width 0.6) (layer "F.Cu") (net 13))
 (segment (start 153 70) (end 151 72) (width 0.6) (layer "F.Cu") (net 13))
 (segment (start 137.6865 84.1865) (end 138.27 84.77) (width 0.6) (layer "F.Cu") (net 6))
 (segment (start 138.27 84.77) (end 139 84.77) (width 0.6) (layer "F.Cu") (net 6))
 (segment (start 141.16 94) (end 141.16 83.904666) (width 0.6) (layer "F.Cu") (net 6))
 (segment (start 154.751388 96.152) (end 143.312 96.152) (width 0.6) (layer "F.Cu") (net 6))
 (segment (start 137.6865 83.058166) (end 137.6865 84.1865) (width 0.6) (layer "F.Cu") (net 6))
 (segment (start 156.012 94.891389) (end 154.751388 96.152) (width 0.6) (layer "F.Cu") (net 6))
 (segment (start 141.16 83.904666) (end 139.929334 82.674) (width 0.6) (layer "F.Cu") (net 6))
 (segment (start 139.929334 82.674) (end 138.070666 82.674) (width 0.6) (layer "F.Cu") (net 6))
 (segment (start 143.312 96.152) (end 141.16 94) (width 0.6) (layer "F.Cu") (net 6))
 (segment (start 151 74.8) (end 156.012 79.812) (width 0.6) (layer "F.Cu") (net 6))
 (segment (start 138.070666 82.674) (end 137.6865 83.058166) (width 0.6) (layer "F.Cu") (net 6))
 (segment (start 156.012 79.812) (end 156.012 94.891389) (width 0.6) (layer "F.Cu") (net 6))
 (segment (start 138.62 94) (end 140.3135 92.3065) (width 0.6) (layer "F.Cu") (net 5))
 (segment (start 140.3135 84.328166) (end 139.485334 83.5) (width 0.6) (layer "F.Cu") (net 5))
 (segment (start 140.3135 92.3065) (end 140.3135 84.328166) (width 0.6) (layer "F.Cu") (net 5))
 (segment (start 139.485334 83.5) (end 139 83.5) (width 0.6) (layer "F.Cu") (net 5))
 (segment (start 146.175 86.04) (end 147.810603 86.04) (width 0.6) (layer "F.Cu") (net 2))
 (segment (start 135.520906 76) (end 129.5 76) (width 0.6) (layer "F.Cu") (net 2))
 (segment (start 146.24 94) (end 142.762 90.522) (width 0.6) (layer "F.Cu") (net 2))
 (segment (start 147.591 95.351) (end 146.24 94) (width 0.6) (layer "F.Cu") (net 2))
 (segment (start 142.762 90.522) (end 142.762 83.241094) (width 0.6) (layer "F.Cu") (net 2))
 (segment (start 155.211 94.559603) (end 154.419603 95.351) (width 0.6) (layer "F.Cu") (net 2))
 (segment (start 154.419603 95.351) (end 147.591 95.351) (width 0.6) (layer "F.Cu") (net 2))
 (segment (start 142.762 83.241094) (end 135.520906 76) (width 0.6) (layer "F.Cu") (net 2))
 (segment (start 155.211 93.440397) (end 155.211 94.559603) (width 0.6) (layer "F.Cu") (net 2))
 (segment (start 147.810603 86.04) (end 155.211 93.440397) (width 0.6) (layer "F.Cu") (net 2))
 (segment (start 137.73888 81.873) (end 136.8855 82.726381) (width 0.6) (layer "F.Cu") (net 7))
 (segment (start 137.73888 81.873) (end 137.738881 81.873) (width 0.6) (layer "F.Cu") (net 7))
 (segment (start 139.597548 81.873) (end 138.402452 81.873) (width 0.6) (layer "F.Cu") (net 7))
 (segment (start 136.8855 84.875213) (end 138.050287 86.04) (width 0.6) (layer "F.Cu") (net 7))
 (segment (start 141.961 84.961) (end 141.961 84.236452) (width 0.6) (layer "F.Cu") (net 7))
 (segment (start 138.050287 86.04) (end 139 86.04) (width 0.6) (layer "F.Cu") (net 7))
 (segment (start 143.7 94) (end 143.7 93.2) (width 0.6) (layer "F.Cu") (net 7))
 (segment (start 140.261119 81.873) (end 139.597548 81.873) (width 0.6) (layer "F.Cu") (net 7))
 (segment (start 136.8855 83.389952) (end 136.8855 83.854714) (width 0.6) (layer "F.Cu") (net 7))
 (segment (start 140.730334 82.342215) (end 140.26112 81.873) (width 0.6) (layer "F.Cu") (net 7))
 (segment (start 140.26112 81.873) (end 140.261119 81.873) (width 0.6) (layer "F.Cu") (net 7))
 (segment (start 141.961 83.57288) (end 140.730334 82.342215) (width 0.6) (layer "F.Cu") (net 7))
 (segment (start 141.961 83.572881) (end 141.961 83.57288) (width 0.6) (layer "F.Cu") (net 7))
 (segment (start 141.961 84.236452) (end 141.961 83.572881) (width 0.6) (layer "F.Cu") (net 7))
 (segment (start 138.402452 81.873) (end 137.738881 81.873) (width 0.6) (layer "F.Cu") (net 7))
 (segment (start 136.8855 83.854714) (end 136.8855 84.518285) (width 0.6) (layer "F.Cu") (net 7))
 (segment (start 136.8855 84.518286) (end 136.8855 84.875213) (width 0.6) (layer "F.Cu") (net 7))
 (segment (start 136.8855 84.518285) (end 136.8855 84.518286) (width 0.6) (layer "F.Cu") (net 7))
 (segment (start 143.7 93.2) (end 141.961 91.461) (width 0.6) (layer "F.Cu") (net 7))
 (segment (start 141.961 91.461) (end 141.961 84.961) (width 0.6) (layer "F.Cu") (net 7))
 (segment (start 136.8855 82.726381) (end 136.8855 83.389952) (width 0.6) (layer "F.Cu") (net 7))
 (segment (start 151.32 94) (end 146.175 88.855) (width 0.6) (layer "F.Cu") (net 1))
 (segment (start 146.175 88.855) (end 146.175 87.31) (width 0.6) (layer "F.Cu") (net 1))
 (segment (start 145.27 84.77) (end 146.175 84.77) (width 0.6) (layer "F.Cu") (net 3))
 (segment (start 131.181954 69.951) (end 129.818046 69.951) (width 0.6) (layer "F.Cu") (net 3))
 (segment (start 144.8615 85.1785) (end 145.27 84.77) (width 0.6) (layer "F.Cu") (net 3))
 (segment (start 146.37749 84.77) (end 146.175 84.77) (width 0.2) (layer "F.Cu") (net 3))
 (segment (start 144.8615 90.0815) (end 144.8615 85.1785) (width 0.6) (layer "F.Cu") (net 3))
 (segment (start 129.399 68.468046) (end 130.367046 67.5) (width 0.6) (layer "F.Cu") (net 3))
 (segment (start 129.399 69.531954) (end 129.399 68.468046) (width 0.6) (layer "F.Cu") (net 3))
 (segment (start 130.367046 67.5) (end 142 67.5) (width 0.6) (layer "F.Cu") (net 3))
 (segment (start 146.175 84.77) (end 146.445 84.5) (width 0.2) (layer "F.Cu") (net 3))
 (segment (start 144.8615 85.1785) (end 144.8615 83.630546) (width 0.6) (layer "F.Cu") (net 3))
 (segment (start 148.78 94) (end 144.8615 90.0815) (width 0.6) (layer "F.Cu") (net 3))
 (segment (start 129.818046 69.951) (end 129.399 69.531954) (width 0.6) (layer "F.Cu") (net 3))
 (segment (start 144.8615 83.630546) (end 131.181954 69.951) (width 0.6) (layer "F.Cu") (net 3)))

